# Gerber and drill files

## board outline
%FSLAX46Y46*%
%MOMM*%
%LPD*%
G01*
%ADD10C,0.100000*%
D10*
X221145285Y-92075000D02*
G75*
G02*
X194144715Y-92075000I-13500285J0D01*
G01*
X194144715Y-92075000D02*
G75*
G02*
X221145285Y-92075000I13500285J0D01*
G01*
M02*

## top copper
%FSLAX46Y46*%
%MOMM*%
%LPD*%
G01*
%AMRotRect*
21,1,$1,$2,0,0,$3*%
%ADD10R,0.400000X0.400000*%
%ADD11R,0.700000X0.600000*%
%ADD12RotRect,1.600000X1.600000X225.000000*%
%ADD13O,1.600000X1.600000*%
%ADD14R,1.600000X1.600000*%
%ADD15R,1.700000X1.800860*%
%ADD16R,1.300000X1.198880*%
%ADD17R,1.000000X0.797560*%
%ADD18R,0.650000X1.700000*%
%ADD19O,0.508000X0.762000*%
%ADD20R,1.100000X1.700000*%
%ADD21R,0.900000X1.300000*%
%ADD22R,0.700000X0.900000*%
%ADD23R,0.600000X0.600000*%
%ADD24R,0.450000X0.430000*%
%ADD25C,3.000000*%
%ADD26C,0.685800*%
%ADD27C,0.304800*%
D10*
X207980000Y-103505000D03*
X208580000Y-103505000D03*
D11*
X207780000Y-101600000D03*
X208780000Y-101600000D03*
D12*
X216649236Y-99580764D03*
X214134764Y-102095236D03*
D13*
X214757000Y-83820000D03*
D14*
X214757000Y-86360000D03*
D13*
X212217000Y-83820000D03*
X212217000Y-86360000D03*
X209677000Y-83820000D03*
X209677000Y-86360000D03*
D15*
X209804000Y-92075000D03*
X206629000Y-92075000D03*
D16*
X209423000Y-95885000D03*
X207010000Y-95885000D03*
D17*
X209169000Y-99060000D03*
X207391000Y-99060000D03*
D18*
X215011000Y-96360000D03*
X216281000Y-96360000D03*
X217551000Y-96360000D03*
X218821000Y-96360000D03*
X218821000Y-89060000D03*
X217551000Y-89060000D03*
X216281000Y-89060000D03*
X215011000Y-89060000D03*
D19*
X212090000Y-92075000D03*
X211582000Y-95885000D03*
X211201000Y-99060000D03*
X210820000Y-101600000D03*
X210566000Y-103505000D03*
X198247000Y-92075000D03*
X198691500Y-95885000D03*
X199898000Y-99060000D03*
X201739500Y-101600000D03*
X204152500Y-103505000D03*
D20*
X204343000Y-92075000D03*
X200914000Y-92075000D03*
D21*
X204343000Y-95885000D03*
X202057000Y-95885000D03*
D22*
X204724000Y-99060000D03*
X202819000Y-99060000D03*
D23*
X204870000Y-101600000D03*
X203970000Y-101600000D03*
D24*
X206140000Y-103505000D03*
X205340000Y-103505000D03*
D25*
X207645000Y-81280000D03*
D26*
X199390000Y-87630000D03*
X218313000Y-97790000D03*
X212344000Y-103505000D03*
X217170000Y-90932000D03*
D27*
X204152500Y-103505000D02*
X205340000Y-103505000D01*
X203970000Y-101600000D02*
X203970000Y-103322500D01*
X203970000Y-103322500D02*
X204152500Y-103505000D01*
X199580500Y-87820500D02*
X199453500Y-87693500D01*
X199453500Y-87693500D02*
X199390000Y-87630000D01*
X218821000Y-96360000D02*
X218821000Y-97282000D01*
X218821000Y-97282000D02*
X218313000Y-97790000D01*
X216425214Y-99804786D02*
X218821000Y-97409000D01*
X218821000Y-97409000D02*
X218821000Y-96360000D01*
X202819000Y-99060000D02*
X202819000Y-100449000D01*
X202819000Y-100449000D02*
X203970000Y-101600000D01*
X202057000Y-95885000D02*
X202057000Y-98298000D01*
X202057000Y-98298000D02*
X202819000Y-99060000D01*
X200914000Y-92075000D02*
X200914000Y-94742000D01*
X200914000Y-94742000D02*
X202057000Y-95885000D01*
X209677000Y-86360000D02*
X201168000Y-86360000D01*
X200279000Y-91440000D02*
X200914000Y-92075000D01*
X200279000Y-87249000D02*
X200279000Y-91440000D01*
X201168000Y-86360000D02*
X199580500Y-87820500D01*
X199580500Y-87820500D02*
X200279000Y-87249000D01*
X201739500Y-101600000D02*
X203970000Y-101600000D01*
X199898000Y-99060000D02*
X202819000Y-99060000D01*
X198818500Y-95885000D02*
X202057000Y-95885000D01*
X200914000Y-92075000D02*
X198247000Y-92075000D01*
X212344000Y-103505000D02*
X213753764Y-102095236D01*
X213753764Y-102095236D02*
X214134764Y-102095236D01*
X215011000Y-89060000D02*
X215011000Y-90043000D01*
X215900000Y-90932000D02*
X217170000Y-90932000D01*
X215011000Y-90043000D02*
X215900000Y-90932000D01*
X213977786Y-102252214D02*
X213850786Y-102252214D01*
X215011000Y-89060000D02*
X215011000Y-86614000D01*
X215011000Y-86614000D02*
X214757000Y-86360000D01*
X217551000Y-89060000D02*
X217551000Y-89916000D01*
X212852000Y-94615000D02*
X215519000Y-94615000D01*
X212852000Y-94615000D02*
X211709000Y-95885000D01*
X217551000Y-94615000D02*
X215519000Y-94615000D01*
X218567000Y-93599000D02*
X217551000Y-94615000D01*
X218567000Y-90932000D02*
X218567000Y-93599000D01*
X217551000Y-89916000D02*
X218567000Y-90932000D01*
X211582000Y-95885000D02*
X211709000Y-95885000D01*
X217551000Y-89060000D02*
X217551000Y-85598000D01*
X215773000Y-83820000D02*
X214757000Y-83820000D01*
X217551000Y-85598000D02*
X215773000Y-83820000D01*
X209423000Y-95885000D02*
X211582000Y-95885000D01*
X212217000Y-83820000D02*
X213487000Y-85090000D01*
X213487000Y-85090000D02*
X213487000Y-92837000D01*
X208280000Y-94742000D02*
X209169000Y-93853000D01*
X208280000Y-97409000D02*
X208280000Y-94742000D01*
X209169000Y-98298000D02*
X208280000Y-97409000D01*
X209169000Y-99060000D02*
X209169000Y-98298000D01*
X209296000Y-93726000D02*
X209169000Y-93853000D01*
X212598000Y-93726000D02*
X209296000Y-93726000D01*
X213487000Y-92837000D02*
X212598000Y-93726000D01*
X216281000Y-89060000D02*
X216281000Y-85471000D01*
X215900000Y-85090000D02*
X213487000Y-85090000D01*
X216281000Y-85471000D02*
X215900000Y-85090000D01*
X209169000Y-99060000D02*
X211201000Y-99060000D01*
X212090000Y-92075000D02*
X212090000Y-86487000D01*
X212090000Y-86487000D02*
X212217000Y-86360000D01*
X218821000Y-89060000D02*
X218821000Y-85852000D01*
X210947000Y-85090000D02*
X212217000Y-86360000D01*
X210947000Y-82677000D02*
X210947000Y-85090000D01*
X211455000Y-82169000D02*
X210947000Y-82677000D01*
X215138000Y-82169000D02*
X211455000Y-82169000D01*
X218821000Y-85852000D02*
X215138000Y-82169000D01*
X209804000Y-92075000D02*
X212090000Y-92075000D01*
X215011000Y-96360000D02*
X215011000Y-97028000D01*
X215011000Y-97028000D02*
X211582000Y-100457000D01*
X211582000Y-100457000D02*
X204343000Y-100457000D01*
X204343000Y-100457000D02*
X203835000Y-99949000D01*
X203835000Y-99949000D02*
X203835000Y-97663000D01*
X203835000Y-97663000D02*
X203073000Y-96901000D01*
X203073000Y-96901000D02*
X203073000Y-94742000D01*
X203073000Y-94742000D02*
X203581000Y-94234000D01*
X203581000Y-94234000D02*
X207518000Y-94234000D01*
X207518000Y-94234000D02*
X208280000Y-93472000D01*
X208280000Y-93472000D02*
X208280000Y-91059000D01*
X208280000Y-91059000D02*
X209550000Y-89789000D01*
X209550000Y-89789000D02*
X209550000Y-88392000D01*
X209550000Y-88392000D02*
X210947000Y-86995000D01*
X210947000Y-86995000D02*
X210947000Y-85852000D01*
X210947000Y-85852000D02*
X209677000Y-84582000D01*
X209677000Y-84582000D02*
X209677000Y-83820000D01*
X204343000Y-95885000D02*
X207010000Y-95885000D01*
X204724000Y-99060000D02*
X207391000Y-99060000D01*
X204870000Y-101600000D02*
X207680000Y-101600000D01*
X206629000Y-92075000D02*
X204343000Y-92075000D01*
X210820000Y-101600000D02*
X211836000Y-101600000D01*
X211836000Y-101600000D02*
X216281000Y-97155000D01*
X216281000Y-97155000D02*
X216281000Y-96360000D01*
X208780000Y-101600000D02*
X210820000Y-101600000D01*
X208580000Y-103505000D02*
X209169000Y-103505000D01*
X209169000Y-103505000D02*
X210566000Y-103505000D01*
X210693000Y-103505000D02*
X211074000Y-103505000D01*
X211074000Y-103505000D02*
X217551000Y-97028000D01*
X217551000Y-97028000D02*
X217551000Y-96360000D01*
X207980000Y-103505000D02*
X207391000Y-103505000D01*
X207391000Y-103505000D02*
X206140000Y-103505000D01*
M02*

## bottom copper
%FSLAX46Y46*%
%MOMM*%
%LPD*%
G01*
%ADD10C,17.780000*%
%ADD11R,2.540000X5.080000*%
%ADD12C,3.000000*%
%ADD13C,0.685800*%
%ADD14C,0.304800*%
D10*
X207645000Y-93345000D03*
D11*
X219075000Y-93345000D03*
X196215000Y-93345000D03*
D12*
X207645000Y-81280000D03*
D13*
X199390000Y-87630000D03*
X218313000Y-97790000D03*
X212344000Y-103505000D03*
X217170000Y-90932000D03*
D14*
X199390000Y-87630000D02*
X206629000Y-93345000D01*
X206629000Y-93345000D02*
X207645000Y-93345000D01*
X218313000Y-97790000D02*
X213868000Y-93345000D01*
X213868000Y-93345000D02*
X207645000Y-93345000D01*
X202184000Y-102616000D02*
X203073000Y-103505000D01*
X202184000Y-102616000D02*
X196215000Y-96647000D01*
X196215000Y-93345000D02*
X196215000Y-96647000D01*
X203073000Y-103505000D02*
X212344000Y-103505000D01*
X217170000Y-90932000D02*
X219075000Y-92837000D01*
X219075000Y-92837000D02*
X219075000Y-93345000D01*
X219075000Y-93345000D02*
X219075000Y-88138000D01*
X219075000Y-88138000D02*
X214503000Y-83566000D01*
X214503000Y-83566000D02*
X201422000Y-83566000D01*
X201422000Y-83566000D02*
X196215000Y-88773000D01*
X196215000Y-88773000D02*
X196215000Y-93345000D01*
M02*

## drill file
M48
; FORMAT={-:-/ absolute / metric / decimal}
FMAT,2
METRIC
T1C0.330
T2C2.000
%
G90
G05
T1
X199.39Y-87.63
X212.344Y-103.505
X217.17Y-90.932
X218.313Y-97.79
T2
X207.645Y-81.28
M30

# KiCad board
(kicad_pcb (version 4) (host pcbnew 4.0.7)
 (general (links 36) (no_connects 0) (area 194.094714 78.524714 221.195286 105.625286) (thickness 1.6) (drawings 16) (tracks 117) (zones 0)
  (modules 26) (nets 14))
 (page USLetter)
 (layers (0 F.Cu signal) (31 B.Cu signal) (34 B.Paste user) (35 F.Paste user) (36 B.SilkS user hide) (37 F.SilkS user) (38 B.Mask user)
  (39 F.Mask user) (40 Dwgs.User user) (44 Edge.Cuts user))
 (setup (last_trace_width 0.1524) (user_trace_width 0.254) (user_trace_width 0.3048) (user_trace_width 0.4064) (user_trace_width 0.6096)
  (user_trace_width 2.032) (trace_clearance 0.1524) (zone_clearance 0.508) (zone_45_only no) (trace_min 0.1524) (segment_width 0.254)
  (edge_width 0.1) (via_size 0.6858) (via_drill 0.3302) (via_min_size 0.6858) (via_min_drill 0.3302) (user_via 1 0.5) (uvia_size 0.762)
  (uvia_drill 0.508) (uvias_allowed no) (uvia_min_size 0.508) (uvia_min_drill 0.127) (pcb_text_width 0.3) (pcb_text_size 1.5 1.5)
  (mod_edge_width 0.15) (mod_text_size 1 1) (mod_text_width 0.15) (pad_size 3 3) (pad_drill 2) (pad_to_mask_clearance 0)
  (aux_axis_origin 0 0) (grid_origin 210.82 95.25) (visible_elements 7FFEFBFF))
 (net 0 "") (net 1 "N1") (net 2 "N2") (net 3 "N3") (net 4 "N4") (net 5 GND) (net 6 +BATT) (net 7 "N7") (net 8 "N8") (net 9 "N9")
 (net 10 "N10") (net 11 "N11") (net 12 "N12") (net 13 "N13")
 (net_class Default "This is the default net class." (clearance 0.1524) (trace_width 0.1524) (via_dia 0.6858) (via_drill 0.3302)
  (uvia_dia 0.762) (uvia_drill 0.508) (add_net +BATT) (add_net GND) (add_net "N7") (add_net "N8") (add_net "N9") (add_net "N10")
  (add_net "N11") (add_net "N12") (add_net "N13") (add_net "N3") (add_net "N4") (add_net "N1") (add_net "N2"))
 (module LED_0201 (layer F.Cu) (at 208.28 103.505)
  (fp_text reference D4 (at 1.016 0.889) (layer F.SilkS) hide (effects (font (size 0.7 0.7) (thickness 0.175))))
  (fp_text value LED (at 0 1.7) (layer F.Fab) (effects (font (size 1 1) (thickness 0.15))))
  (pad 1 smd rect (at -0.3 0) (size 0.4 0.4) (layers F.Cu F.Paste F.Mask) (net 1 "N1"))
  (pad 2 smd rect (at 0.3 0) (size 0.4 0.4) (layers F.Cu F.Paste F.Mask) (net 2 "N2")))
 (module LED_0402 (layer F.Cu) (at 208.28 101.6)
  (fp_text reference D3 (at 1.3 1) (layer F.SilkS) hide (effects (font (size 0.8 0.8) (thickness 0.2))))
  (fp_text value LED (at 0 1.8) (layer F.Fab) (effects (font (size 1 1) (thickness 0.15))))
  (pad 1 smd rect (at -0.5 0) (size 0.7 0.6) (layers F.Cu F.Paste F.Mask) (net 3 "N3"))
  (pad 2 smd rect (at 0.5 0) (size 0.7 0.6) (layers F.Cu F.Paste F.Mask) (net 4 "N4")))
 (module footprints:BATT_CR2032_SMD (layer B.Cu) (at 207.645 93.345 180)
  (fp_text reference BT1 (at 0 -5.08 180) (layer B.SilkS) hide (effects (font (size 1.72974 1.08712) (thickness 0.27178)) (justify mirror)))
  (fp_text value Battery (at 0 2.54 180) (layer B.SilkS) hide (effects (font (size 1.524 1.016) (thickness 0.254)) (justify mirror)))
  (pad 2 smd circle (at 0 0 180) (size 17.78 17.78) (layers B.Cu B.Paste B.Mask) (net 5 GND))
  (pad 1 smd rect (at -11.43 0 180) (size 2.54 5.08) (layers B.Cu B.Paste B.Mask) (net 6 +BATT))
  (pad 1 smd rect (at 11.43 0 180) (size 2.54 5.08) (layers B.Cu B.Paste B.Mask) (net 6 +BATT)))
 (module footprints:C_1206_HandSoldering (layer F.Cu) (at 215.392 100.838 225)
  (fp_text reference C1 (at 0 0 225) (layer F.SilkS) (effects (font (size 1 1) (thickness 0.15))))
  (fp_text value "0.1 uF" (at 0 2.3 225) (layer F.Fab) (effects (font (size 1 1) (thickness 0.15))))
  (pad 1 smd rect (at -1.778 0 225) (size 1.6 1.6) (layers F.Cu F.Paste F.Mask) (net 5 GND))
  (pad 2 smd rect (at 1.778 0 225) (size 1.6 1.6) (layers F.Cu F.Paste F.Mask) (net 6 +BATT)))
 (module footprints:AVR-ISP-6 (layer F.Cu) (at 214.757 83.82 270)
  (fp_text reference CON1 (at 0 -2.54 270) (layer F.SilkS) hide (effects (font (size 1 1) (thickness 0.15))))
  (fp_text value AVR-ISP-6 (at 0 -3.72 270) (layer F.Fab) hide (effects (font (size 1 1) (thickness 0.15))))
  (pad 1 smd oval (at 0 0 270) (size 1.6 1.6) (layers F.Cu F.Paste F.Mask) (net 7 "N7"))
  (pad 2 smd rect (at 2.54 0 270) (size 1.6 1.6) (layers F.Cu F.Paste F.Mask) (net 6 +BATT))
  (pad 3 smd oval (at 0 2.54 270) (size 1.6 1.6) (layers F.Cu F.Paste F.Mask) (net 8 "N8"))
  (pad 4 smd oval (at 2.54 2.54 270) (size 1.6 1.6) (layers F.Cu F.Paste F.Mask) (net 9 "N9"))
  (pad 5 smd oval (at 0 5.08 270) (size 1.6 1.6) (layers F.Cu F.Paste F.Mask) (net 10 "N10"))
  (pad 6 smd oval (at 2.54 5.08 270) (size 1.6 1.6) (layers F.Cu F.Paste F.Mask) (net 5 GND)))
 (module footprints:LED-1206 (layer F.Cu) (at 208.28 92.075)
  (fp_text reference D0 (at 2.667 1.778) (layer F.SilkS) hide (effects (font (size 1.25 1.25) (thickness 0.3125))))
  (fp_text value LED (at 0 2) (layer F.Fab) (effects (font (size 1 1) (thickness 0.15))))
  (pad 2 smd rect (at 1.524 0 180) (size 1.7 1.80086) (layers F.Cu F.Paste F.Mask) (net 9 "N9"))
  (pad 1 smd rect (at -1.651 0 180) (size 1.7 1.80086) (layers F.Cu F.Paste F.Mask) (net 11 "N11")))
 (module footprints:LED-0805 (layer F.Cu) (at 208.28 95.885)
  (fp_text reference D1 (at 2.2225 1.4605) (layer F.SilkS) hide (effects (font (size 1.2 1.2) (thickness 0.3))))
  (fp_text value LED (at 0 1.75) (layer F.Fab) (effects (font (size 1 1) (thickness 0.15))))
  (pad 2 smd rect (at 1.143 0 180) (size 1.3 1.19888) (layers F.Cu F.Paste F.Mask) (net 7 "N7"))
  (pad 1 smd rect (at -1.27 0 180) (size 1.3 1.19888) (layers F.Cu F.Paste F.Mask) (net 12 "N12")))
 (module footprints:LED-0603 (layer F.Cu) (at 208.28 99.06)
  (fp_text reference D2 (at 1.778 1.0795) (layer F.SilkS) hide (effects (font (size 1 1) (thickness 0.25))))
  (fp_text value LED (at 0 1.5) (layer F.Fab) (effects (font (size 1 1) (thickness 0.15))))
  (pad 2 smd rect (at 0.889 0 180) (size 1 0.79756) (layers F.Cu F.Paste F.Mask) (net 8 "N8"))
  (pad 1 smd rect (at -0.889 0 180) (size 1 0.79756) (layers F.Cu F.Paste F.Mask) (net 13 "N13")))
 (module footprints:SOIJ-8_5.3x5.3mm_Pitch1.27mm (layer F.Cu) (at 216.916 92.71 90)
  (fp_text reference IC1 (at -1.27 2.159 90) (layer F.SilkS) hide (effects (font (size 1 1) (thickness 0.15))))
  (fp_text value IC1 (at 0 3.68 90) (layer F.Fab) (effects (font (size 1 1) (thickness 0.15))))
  (pad 1 smd rect (at -3.65 -1.905 90) (size 1.7 0.65) (layers F.Cu F.Paste F.Mask) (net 10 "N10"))
  (pad 2 smd rect (at -3.65 -0.635 90) (size 1.7 0.65) (layers F.Cu F.Paste F.Mask) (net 4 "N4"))
  (pad 3 smd rect (at -3.65 0.635 90) (size 1.7 0.65) (layers F.Cu F.Paste F.Mask) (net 2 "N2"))
  (pad 4 smd rect (at -3.65 1.905 90) (size 1.7 0.65) (layers F.Cu F.Paste F.Mask) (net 5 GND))
  (pad 5 smd rect (at 3.65 1.905 90) (size 1.7 0.65) (layers F.Cu F.Paste F.Mask) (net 9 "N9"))
  (pad 6 smd rect (at 3.65 0.635 90) (size 1.7 0.65) (layers F.Cu F.Paste F.Mask) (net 7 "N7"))
  (pad 7 smd rect (at 3.65 -0.635 90) (size 1.7 0.65) (layers F.Cu F.Paste F.Mask) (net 8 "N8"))
  (pad 8 smd rect (at 3.65 -1.905 90) (size 1.7 0.65) (layers F.Cu F.Paste F.Mask) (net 6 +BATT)))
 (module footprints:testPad (layer F.Cu) (at 212.09 92.075)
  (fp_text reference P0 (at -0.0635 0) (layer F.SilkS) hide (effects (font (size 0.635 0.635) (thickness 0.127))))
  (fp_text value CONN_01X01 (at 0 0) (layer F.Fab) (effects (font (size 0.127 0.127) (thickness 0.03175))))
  (pad 1 smd oval (at 0 0) (size 0.508 0.762) (layers F.Cu F.Paste F.Mask) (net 9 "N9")))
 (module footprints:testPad (layer F.Cu) (at 211.582 95.885)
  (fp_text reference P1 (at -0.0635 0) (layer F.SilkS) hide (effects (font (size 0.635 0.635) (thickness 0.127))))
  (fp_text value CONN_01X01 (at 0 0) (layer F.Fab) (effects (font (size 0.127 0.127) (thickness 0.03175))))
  (pad 1 smd oval (at 0 0) (size 0.508 0.762) (layers F.Cu F.Paste F.Mask) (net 7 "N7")))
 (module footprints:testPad (layer F.Cu) (at 211.201 99.06)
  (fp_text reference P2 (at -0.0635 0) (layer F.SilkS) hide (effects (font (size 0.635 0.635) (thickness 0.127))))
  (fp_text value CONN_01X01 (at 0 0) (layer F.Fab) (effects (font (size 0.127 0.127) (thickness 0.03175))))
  (pad 1 smd oval (at 0 0) (size 0.508 0.762) (layers F.Cu F.Paste F.Mask) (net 8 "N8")))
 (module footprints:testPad (layer F.Cu) (at 210.82 101.6)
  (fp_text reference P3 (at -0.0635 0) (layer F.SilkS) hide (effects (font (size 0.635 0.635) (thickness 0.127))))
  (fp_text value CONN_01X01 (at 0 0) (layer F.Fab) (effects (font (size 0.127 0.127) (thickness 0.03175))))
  (pad 1 smd oval (at 0 0) (size 0.508 0.762) (layers F.Cu F.Paste F.Mask) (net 4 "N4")))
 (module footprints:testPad (layer F.Cu) (at 210.566 103.505)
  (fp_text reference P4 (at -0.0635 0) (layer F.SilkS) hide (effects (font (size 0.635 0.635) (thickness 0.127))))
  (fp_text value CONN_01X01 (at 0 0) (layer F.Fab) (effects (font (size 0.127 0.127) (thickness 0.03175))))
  (pad 1 smd oval (at 0 0) (size 0.508 0.762) (layers F.Cu F.Paste F.Mask) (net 2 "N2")))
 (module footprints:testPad (layer F.Cu) (at 198.247 92.075)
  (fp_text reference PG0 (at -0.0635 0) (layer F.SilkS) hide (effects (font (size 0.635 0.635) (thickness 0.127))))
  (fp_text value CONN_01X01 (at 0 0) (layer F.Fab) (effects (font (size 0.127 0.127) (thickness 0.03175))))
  (pad 1 smd oval (at 0 0) (size 0.508 0.762) (layers F.Cu F.Paste F.Mask) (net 5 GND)))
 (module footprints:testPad (layer F.Cu) (at 198.6915 95.885)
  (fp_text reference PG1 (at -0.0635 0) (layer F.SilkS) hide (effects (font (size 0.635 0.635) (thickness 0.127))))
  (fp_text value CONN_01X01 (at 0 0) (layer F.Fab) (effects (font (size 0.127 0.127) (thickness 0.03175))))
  (pad 1 smd oval (at 0 0) (size 0.508 0.762) (layers F.Cu F.Paste F.Mask) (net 5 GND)))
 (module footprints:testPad (layer F.Cu) (at 199.898 99.06)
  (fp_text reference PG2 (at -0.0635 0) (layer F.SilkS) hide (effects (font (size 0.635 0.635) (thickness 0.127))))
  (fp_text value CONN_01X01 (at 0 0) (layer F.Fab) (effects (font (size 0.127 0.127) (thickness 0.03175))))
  (pad 1 smd oval (at 0 0) (size 0.508 0.762) (layers F.Cu F.Paste F.Mask) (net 5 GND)))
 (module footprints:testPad (layer F.Cu) (at 201.7395 101.6)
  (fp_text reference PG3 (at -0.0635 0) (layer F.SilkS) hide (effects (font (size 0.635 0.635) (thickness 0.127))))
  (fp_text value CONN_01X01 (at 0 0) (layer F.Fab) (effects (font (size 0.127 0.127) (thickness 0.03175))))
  (pad 1 smd oval (at 0 0) (size 0.508 0.762) (layers F.Cu F.Paste F.Mask) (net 5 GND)))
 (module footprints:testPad (layer F.Cu) (at 204.1525 103.505)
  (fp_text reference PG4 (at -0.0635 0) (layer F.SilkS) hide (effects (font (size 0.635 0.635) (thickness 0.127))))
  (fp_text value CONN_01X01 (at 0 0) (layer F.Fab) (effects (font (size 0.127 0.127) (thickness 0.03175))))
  (pad 1 smd oval (at 0 0) (size 0.508 0.762) (layers F.Cu F.Paste F.Mask) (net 5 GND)))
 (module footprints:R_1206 (layer F.Cu) (at 202.565 92.075 180)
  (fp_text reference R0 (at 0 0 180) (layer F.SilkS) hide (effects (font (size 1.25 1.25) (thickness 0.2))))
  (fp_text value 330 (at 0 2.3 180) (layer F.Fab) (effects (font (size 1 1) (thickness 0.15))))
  (pad 1 smd rect (at -1.778 0 180) (size 1.1 1.7) (layers F.Cu F.Paste F.Mask) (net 11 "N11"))
  (pad 2 smd rect (at 1.651 0 180) (size 1.1 1.7) (layers F.Cu F.Paste F.Mask) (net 5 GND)))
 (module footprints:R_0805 (layer F.Cu) (at 203.2 95.885 180)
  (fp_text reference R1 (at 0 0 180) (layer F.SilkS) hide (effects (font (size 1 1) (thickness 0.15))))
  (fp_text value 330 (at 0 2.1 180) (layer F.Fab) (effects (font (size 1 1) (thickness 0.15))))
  (pad 1 smd rect (at -1.143 0 180) (size 0.9 1.3) (layers F.Cu F.Paste F.Mask) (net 12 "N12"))
  (pad 2 smd rect (at 1.143 0 180) (size 0.9 1.3) (layers F.Cu F.Paste F.Mask) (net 5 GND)))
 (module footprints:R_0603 (layer F.Cu) (at 203.835 99.06 180)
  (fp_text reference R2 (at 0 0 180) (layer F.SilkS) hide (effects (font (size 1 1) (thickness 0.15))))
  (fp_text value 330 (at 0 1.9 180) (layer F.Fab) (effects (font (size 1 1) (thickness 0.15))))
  (pad 1 smd rect (at -0.889 0 180) (size 0.7 0.9) (layers F.Cu F.Paste F.Mask) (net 13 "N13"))
  (pad 2 smd rect (at 1.016 0 180) (size 0.7 0.9) (layers F.Cu F.Paste F.Mask) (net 5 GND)))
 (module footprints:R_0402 (layer F.Cu) (at 204.47 101.6 180)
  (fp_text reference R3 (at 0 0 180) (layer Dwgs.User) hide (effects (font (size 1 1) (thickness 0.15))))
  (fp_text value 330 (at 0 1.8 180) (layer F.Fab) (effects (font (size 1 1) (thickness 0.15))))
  (pad 1 smd rect (at -0.4 0 180) (size 0.6 0.6) (layers F.Cu F.Paste F.Mask) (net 3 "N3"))
  (pad 2 smd rect (at 0.5 0 180) (size 0.6 0.6) (layers F.Cu F.Paste F.Mask) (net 5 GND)))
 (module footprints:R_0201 (layer F.Cu) (at 205.74 103.505 180)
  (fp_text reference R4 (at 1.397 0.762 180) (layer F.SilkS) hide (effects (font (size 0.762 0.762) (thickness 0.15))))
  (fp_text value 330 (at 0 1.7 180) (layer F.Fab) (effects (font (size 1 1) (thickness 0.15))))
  (pad 1 smd rect (at -0.4 0 180) (size 0.45 0.43) (layers F.Cu F.Paste F.Mask) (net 1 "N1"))
  (pad 2 smd rect (at 0.4 0 180) (size 0.45 0.43) (layers F.Cu F.Paste F.Mask) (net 5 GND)))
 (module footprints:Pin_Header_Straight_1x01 (layer F.Cu) (at 207.645 81.28)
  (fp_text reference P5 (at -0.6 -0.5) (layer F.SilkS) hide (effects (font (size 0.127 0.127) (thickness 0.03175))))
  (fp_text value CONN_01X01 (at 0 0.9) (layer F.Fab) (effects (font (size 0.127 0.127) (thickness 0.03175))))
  (pad 1 thru_hole circle (at 0 0) (size 3 3) (drill 2) (layers *.Cu *.Mask)))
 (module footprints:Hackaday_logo (layer F.Cu) (at 202.52 86.25)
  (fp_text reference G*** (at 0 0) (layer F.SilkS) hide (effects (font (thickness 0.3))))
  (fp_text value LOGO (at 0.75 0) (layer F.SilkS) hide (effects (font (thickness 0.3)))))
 (gr_circle (center 207.645 92.075) (end 197.485 83.185) (layer Edge.Cuts) (width 0.1))
 (segment (start 204.1525 103.505) (end 205.34 103.505) (width 0.3048) (layer F.Cu) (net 5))
 (segment (start 203.97 101.6) (end 203.97 103.3225) (width 0.3048) (layer F.Cu) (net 5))
 (segment (start 203.97 103.3225) (end 204.1525 103.505) (width 0.3048) (layer F.Cu) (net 5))
 (segment (start 199.5805 87.8205) (end 199.4535 87.6935) (width 0.3048) (layer F.Cu) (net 5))
 (segment (start 199.39 87.63) (end 206.629 93.345) (width 0.3048) (layer B.Cu) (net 5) (status 20))
 (via (at 199.39 87.63) (size 0.6858) (drill 0.3302) (layers F.Cu B.Cu) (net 5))
 (segment (start 199.4535 87.6935) (end 199.39 87.63) (width 0.3048) (layer F.Cu) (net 5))
 (segment (start 206.629 93.345) (end 207.645 93.345) (width 0.3048) (layer B.Cu) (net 5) (status 30))
 (segment (start 218.821 96.36) (end 218.821 97.282) (width 0.3048) (layer F.Cu) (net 5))
 (segment (start 218.313 97.79) (end 213.868 93.345) (width 0.3048) (layer B.Cu) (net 5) (status 20))
 (via (at 218.313 97.79) (size 0.6858) (drill 0.3302) (layers F.Cu B.Cu) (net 5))
 (segment (start 218.821 97.282) (end 218.313 97.79) (width 0.3048) (layer F.Cu) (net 5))
 (segment (start 213.868 93.345) (end 207.645 93.345) (width 0.3048) (layer B.Cu) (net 5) (status 30))
 (segment (start 216.425214 99.804786) (end 218.821 97.409) (width 0.3048) (layer F.Cu) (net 5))
 (segment (start 218.821 97.409) (end 218.821 96.36) (width 0.3048) (layer F.Cu) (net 5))
 (segment (start 202.819 99.06) (end 202.819 100.449) (width 0.3048) (layer F.Cu) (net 5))
 (segment (start 202.819 100.449) (end 203.97 101.6) (width 0.3048) (layer F.Cu) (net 5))
 (segment (start 202.057 95.885) (end 202.057 98.298) (width 0.3048) (layer F.Cu) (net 5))
 (segment (start 202.057 98.298) (end 202.819 99.06) (width 0.3048) (layer F.Cu) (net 5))
 (segment (start 200.914 92.075) (end 200.914 94.742) (width 0.3048) (layer F.Cu) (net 5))
 (segment (start 200.914 94.742) (end 202.057 95.885) (width 0.3048) (layer F.Cu) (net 5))
 (segment (start 209.677 86.36) (end 201.168 86.36) (width 0.3048) (layer F.Cu) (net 5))
 (segment (start 200.279 91.44) (end 200.914 92.075) (width 0.3048) (layer F.Cu) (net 5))
 (segment (start 200.279 87.249) (end 200.279 91.44) (width 0.3048) (layer F.Cu) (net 5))
 (segment (start 201.168 86.36) (end 199.5805 87.8205) (width 0.3048) (layer F.Cu) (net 5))
 (segment (start 199.5805 87.8205) (end 200.279 87.249) (width 0.3048) (layer F.Cu) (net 5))
 (segment (start 201.7395 101.6) (end 203.97 101.6) (width 0.3048) (layer F.Cu) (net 5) (status 10))
 (segment (start 199.898 99.06) (end 202.819 99.06) (width 0.3048) (layer F.Cu) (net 5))
 (segment (start 198.8185 95.885) (end 202.057 95.885) (width 0.3048) (layer F.Cu) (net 5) (status 10))
 (segment (start 200.914 92.075) (end 198.247 92.075) (width 0.3048) (layer F.Cu) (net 5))
 (segment (start 202.184 102.616) (end 203.073 103.505) (width 0.3048) (layer B.Cu) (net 6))
 (segment (start 202.184 102.616) (end 196.215 96.647) (width 0.3048) (layer B.Cu) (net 6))
 (segment (start 196.215 93.345) (end 196.215 96.647) (width 0.3048) (layer B.Cu) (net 6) (status 10))
 (segment (start 212.344 103.505) (end 213.753764 102.095236) (width 0.3048) (layer F.Cu) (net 6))
 (via (at 212.344 103.505) (size 0.6858) (drill 0.3302) (layers F.Cu B.Cu) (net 6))
 (segment (start 203.073 103.505) (end 212.344 103.505) (width 0.3048) (layer B.Cu) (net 6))
 (segment (start 213.753764 102.095236) (end 214.134764 102.095236) (width 0.3048) (layer F.Cu) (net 6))
 (segment (start 215.011 89.06) (end 215.011 90.043) (width 0.3048) (layer F.Cu) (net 6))
 (segment (start 217.17 90.932) (end 219.075 92.837) (width 0.3048) (layer B.Cu) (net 6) (status 20))
 (via (at 217.17 90.932) (size 0.6858) (drill 0.3302) (layers F.Cu B.Cu) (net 6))
 (segment (start 215.9 90.932) (end 217.17 90.932) (width 0.3048) (layer F.Cu) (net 6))
 (segment (start 215.011 90.043) (end 215.9 90.932) (width 0.3048) (layer F.Cu) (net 6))
 (segment (start 219.075 92.837) (end 219.075 93.345) (width 0.3048) (layer B.Cu) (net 6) (status 30))
 (segment (start 219.075 93.345) (end 219.075 88.138) (width 0.3048) (layer B.Cu) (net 6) (status 10))
 (segment (start 219.075 88.138) (end 214.503 83.566) (width 0.3048) (layer B.Cu) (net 6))
 (segment (start 214.503 83.566) (end 201.422 83.566) (width 0.3048) (layer B.Cu) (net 6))
 (segment (start 201.422 83.566) (end 196.215 88.773) (width 0.3048) (layer B.Cu) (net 6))
 (segment (start 196.215 88.773) (end 196.215 93.345) (width 0.3048) (layer B.Cu) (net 6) (status 20))
 (segment (start 213.977786 102.252214) (end 213.850786 102.252214) (width 0.3048) (layer F.Cu) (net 6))
 (segment (start 215.011 89.06) (end 215.011 86.614) (width 0.3048) (layer F.Cu) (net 6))
 (segment (start 215.011 86.614) (end 214.757 86.36) (width 0.3048) (layer F.Cu) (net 6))
 (segment (start 217.551 89.06) (end 217.551 89.916) (width 0.3048) (layer F.Cu) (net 7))
 (segment (start 212.852 94.615) (end 215.519 94.615) (width 0.3048) (layer F.Cu) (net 7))
 (segment (start 212.852 94.615) (end 211.709 95.885) (width 0.3048) (layer F.Cu) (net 7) (status 20))
 (segment (start 217.551 94.615) (end 215.519 94.615) (width 0.3048) (layer F.Cu) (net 7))
 (segment (start 218.567 93.599) (end 217.551 94.615) (width 0.3048) (layer F.Cu) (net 7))
 (segment (start 218.567 90.932) (end 218.567 93.599) (width 0.3048) (layer F.Cu) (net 7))
 (segment (start 217.551 89.916) (end 218.567 90.932) (width 0.3048) (layer F.Cu) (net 7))
 (segment (start 211.582 95.885) (end 211.709 95.885) (width 0.3048) (layer F.Cu) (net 7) (status 30))
 (segment (start 217.551 89.06) (end 217.551 85.598) (width 0.3048) (layer F.Cu) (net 7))
 (segment (start 215.773 83.82) (end 214.757 83.82) (width 0.3048) (layer F.Cu) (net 7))
 (segment (start 217.551 85.598) (end 215.773 83.82) (width 0.3048) (layer F.Cu) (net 7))
 (segment (start 209.423 95.885) (end 211.582 95.885) (width 0.3048) (layer F.Cu) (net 7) (status 20))
 (segment (start 212.217 83.82) (end 213.487 85.09) (width 0.3048) (layer F.Cu) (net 8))
 (segment (start 213.487 85.09) (end 213.487 92.837) (width 0.3048) (layer F.Cu) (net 8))
 (segment (start 208.28 94.742) (end 209.169 93.853) (width 0.3048) (layer F.Cu) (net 8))
 (segment (start 208.28 97.409) (end 208.28 94.742) (width 0.3048) (layer F.Cu) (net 8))
 (segment (start 209.169 98.298) (end 208.28 97.409) (width 0.3048) (layer F.Cu) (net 8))
 (segment (start 209.169 99.06) (end 209.169 98.298) (width 0.3048) (layer F.Cu) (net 8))
 (segment (start 209.296 93.726) (end 209.169 93.853) (width 0.3048) (layer F.Cu) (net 8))
 (segment (start 212.598 93.726) (end 209.296 93.726) (width 0.3048) (layer F.Cu) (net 8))
 (segment (start 213.487 92.837) (end 212.598 93.726) (width 0.3048) (layer F.Cu) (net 8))
 (segment (start 216.281 89.06) (end 216.281 85.471) (width 0.3048) (layer F.Cu) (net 8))
 (segment (start 215.9 85.09) (end 213.487 85.09) (width 0.3048) (layer F.Cu) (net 8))
 (segment (start 216.281 85.471) (end 215.9 85.09) (width 0.3048) (layer F.Cu) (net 8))
 (segment (start 209.169 99.06) (end 211.201 99.06) (width 0.3048) (layer F.Cu) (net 8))
 (segment (start 212.09 92.075) (end 212.09 86.487) (width 0.3048) (layer F.Cu) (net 9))
 (segment (start 212.09 86.487) (end 212.217 86.36) (width 0.3048) (layer F.Cu) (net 9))
 (segment (start 218.821 89.06) (end 218.821 85.852) (width 0.3048) (layer F.Cu) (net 9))
 (segment (start 210.947 85.09) (end 212.217 86.36) (width 0.3048) (layer F.Cu) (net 9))
 (segment (start 210.947 82.677) (end 210.947 85.09) (width 0.3048) (layer F.Cu) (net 9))
 (segment (start 211.455 82.169) (end 210.947 82.677) (width 0.3048) (layer F.Cu) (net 9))
 (segment (start 215.138 82.169) (end 211.455 82.169) (width 0.3048) (layer F.Cu) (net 9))
 (segment (start 218.821 85.852) (end 215.138 82.169) (width 0.3048) (layer F.Cu) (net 9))
 (segment (start 209.804 92.075) (end 212.09 92.075) (width 0.3048) (layer F.Cu) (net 9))
 (segment (start 215.011 96.36) (end 215.011 97.028) (width 0.3048) (layer F.Cu) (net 10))
 (segment (start 215.011 97.028) (end 211.582 100.457) (width 0.3048) (layer F.Cu) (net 10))
 (segment (start 211.582 100.457) (end 204.343 100.457) (width 0.3048) (layer F.Cu) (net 10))
 (segment (start 204.343 100.457) (end 203.835 99.949) (width 0.3048) (layer F.Cu) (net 10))
 (segment (start 203.835 99.949) (end 203.835 97.663) (width 0.3048) (layer F.Cu) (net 10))
 (segment (start 203.835 97.663) (end 203.073 96.901) (width 0.3048) (layer F.Cu) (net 10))
 (segment (start 203.073 96.901) (end 203.073 94.742) (width 0.3048) (layer F.Cu) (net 10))
 (segment (start 203.073 94.742) (end 203.581 94.234) (width 0.3048) (layer F.Cu) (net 10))
 (segment (start 203.581 94.234) (end 207.518 94.234) (width 0.3048) (layer F.Cu) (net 10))
 (segment (start 207.518 94.234) (end 208.28 93.472) (width 0.3048) (layer F.Cu) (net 10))
 (segment (start 208.28 93.472) (end 208.28 91.059) (width 0.3048) (layer F.Cu) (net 10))
 (segment (start 208.28 91.059) (end 209.55 89.789) (width 0.3048) (layer F.Cu) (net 10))
 (segment (start 209.55 89.789) (end 209.55 88.392) (width 0.3048) (layer F.Cu) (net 10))
 (segment (start 209.55 88.392) (end 210.947 86.995) (width 0.3048) (layer F.Cu) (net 10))
 (segment (start 210.947 86.995) (end 210.947 85.852) (width 0.3048) (layer F.Cu) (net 10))
 (segment (start 210.947 85.852) (end 209.677 84.582) (width 0.3048) (layer F.Cu) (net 10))
 (segment (start 209.677 84.582) (end 209.677 83.82) (width 0.3048) (layer F.Cu) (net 10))
 (segment (start 204.343 95.885) (end 207.01 95.885) (width 0.3048) (layer F.Cu) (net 12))
 (segment (start 204.724 99.06) (end 207.391 99.06) (width 0.3048) (layer F.Cu) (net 13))
 (segment (start 204.87 101.6) (end 207.68 101.6) (width 0.3048) (layer F.Cu) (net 3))
 (segment (start 206.629 92.075) (end 204.343 92.075) (width 0.3048) (layer F.Cu) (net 11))
 (segment (start 210.82 101.6) (end 211.836 101.6) (width 0.3048) (layer F.Cu) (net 4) (status 10))
 (segment (start 211.836 101.6) (end 216.281 97.155) (width 0.3048) (layer F.Cu) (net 4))
 (segment (start 216.281 97.155) (end 216.281 96.36) (width 0.3048) (layer F.Cu) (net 4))
 (segment (start 208.78 101.6) (end 210.82 101.6) (width 0.3048) (layer F.Cu) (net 4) (status 20))
 (segment (start 208.58 103.505) (end 209.169 103.505) (width 0.3048) (layer F.Cu) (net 2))
 (segment (start 209.169 103.505) (end 210.566 103.505) (width 0.3048) (layer F.Cu) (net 2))
 (segment (start 210.693 103.505) (end 211.074 103.505) (width 0.3048) (layer F.Cu) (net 2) (status 10))
 (segment (start 211.074 103.505) (end 217.551 97.028) (width 0.3048) (layer F.Cu) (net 2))
 (segment (start 217.551 97.028) (end 217.551 96.36) (width 0.3048) (layer F.Cu) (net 2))
 (segment (start 207.98 103.505) (end 207.391 103.505) (width 0.3048) (layer F.Cu) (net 1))
 (segment (start 207.391 103.505) (end 206.14 103.505) (width 0.3048) (layer F.Cu) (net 1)))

